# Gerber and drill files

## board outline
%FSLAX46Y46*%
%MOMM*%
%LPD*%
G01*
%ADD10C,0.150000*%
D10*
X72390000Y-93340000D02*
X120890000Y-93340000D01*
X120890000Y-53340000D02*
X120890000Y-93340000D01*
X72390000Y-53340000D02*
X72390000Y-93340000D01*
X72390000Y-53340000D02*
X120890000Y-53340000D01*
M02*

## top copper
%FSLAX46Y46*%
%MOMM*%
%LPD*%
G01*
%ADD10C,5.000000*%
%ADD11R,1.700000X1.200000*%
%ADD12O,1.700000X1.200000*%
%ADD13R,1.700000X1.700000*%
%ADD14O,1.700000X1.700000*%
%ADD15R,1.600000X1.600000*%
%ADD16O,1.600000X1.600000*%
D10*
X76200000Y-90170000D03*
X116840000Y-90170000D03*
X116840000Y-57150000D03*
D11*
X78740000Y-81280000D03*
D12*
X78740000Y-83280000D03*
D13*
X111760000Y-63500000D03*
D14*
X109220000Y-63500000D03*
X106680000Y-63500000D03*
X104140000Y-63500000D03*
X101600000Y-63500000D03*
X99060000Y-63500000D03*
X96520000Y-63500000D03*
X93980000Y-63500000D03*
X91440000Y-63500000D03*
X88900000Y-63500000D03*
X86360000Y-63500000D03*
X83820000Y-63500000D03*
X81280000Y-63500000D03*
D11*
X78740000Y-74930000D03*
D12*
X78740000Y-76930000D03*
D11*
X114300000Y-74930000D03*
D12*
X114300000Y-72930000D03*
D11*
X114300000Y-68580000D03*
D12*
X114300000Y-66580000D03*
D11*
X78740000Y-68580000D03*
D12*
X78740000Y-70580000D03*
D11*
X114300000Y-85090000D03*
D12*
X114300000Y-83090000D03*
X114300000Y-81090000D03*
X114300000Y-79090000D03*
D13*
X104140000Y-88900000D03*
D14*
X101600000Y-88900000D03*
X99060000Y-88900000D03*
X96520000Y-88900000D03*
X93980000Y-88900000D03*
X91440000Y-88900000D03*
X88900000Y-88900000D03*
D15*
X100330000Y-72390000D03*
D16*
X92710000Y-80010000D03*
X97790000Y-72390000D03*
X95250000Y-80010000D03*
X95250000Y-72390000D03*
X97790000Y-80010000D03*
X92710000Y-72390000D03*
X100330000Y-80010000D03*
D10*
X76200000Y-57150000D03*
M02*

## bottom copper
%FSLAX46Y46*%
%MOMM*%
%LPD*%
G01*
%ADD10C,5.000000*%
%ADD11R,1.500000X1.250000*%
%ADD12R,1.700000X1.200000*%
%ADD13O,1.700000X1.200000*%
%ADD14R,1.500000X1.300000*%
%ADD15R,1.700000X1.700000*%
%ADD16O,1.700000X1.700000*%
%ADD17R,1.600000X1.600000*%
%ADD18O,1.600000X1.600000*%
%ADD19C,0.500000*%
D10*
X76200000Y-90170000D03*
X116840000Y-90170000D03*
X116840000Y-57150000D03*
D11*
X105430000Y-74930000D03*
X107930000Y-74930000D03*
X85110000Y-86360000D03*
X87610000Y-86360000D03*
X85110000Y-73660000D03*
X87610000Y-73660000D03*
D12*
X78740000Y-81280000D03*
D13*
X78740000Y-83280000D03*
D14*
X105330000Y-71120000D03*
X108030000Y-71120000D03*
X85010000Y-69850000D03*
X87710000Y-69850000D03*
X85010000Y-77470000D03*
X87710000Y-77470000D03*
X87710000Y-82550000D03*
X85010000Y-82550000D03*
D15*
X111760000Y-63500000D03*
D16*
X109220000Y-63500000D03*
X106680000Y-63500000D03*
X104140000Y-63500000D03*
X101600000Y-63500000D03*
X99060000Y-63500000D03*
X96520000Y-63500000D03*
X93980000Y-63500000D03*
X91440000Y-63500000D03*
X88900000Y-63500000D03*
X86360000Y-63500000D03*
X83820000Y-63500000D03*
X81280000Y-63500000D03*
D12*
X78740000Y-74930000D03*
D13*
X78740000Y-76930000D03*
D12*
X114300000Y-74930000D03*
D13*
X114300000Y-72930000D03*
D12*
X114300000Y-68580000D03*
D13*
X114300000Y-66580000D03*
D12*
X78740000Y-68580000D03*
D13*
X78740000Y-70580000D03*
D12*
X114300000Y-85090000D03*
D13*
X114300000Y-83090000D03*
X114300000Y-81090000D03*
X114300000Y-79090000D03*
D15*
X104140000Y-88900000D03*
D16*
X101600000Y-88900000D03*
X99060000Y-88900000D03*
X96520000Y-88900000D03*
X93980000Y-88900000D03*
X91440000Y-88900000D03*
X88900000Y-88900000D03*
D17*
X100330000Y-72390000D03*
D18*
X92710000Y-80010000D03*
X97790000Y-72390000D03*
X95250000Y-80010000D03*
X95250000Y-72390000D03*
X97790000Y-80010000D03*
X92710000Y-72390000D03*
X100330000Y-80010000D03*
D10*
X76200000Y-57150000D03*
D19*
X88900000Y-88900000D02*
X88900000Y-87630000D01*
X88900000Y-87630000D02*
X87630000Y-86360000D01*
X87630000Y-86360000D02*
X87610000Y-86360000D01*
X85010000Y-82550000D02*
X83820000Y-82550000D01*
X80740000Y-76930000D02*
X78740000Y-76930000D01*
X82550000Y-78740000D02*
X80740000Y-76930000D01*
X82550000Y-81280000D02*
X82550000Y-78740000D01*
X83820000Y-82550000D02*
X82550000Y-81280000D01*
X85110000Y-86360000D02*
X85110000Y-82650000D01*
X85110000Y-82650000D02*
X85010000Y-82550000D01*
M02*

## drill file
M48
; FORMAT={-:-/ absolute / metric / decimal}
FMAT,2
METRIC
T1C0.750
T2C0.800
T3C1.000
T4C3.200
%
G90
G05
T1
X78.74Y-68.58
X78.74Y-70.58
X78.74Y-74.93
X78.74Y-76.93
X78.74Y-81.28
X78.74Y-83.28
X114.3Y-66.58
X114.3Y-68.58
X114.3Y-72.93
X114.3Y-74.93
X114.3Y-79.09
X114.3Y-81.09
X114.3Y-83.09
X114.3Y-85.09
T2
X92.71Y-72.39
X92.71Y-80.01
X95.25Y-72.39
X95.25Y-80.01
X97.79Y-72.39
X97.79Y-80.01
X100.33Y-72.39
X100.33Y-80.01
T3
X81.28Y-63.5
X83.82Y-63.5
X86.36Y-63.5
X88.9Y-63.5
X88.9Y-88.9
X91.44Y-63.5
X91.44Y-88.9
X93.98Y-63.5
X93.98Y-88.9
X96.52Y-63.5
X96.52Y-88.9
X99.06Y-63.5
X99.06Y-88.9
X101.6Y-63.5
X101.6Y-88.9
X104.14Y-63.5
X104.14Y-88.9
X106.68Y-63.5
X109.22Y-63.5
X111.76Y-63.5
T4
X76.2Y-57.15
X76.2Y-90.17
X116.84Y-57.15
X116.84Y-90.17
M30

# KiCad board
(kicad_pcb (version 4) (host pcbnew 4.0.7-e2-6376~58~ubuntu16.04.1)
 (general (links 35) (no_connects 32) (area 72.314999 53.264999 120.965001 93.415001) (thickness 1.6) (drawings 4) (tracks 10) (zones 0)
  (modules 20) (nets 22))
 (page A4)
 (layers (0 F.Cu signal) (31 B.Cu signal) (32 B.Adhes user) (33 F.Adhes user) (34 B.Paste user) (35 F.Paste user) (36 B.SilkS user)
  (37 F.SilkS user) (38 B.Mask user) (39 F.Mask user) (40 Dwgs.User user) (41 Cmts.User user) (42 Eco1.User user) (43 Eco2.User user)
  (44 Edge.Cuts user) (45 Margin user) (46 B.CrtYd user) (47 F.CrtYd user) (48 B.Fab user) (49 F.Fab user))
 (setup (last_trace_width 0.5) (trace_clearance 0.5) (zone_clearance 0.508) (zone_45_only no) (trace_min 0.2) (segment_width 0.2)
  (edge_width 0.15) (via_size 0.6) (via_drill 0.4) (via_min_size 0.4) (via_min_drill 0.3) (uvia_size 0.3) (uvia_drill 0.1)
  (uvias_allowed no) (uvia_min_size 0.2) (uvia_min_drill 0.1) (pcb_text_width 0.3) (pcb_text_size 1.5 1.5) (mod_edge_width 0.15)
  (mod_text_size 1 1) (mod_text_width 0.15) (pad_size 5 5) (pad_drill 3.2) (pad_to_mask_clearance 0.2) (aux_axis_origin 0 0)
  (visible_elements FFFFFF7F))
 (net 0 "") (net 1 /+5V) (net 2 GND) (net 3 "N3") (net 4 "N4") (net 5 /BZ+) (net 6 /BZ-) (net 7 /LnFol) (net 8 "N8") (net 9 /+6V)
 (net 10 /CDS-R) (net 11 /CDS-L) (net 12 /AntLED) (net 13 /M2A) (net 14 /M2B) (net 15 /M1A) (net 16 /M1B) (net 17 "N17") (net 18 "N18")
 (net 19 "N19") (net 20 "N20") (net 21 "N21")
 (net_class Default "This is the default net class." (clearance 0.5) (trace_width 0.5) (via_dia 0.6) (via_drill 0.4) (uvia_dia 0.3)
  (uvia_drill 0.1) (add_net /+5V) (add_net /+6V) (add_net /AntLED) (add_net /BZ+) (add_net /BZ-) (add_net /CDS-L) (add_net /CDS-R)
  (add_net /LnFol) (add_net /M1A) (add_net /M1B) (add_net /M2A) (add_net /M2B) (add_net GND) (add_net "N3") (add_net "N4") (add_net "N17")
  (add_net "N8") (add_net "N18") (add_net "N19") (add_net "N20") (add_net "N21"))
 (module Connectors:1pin (layer F.Cu) (at 76.2 90.17)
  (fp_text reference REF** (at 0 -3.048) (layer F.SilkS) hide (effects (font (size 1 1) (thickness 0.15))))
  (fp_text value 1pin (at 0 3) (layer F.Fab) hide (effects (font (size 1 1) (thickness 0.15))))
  (pad 1 thru_hole circle (at 0 0) (size 5 5) (drill 3.2) (layers *.Cu *.Mask)))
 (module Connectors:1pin (layer F.Cu) (at 116.84 90.17)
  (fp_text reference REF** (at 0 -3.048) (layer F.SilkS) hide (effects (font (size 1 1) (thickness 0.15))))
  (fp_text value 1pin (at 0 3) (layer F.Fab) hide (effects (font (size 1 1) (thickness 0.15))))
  (pad 1 thru_hole circle (at 0 0) (size 5 5) (drill 3.2) (layers *.Cu *.Mask)))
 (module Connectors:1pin (layer F.Cu) (at 116.84 57.15)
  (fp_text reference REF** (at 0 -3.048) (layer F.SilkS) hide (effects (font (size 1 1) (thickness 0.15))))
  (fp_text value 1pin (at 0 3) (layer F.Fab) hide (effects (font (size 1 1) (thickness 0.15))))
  (pad 1 thru_hole circle (at 0 0) (size 5 5) (drill 3.2) (layers *.Cu *.Mask)))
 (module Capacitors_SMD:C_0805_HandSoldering (layer B.Cu) (at 106.68 74.93)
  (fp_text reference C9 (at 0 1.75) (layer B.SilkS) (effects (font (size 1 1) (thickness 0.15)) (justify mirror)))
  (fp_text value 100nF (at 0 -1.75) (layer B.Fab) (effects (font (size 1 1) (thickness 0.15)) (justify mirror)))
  (pad 1 smd rect (at -1.25 0) (size 1.5 1.25) (layers B.Cu B.Paste B.Mask) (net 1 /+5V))
  (pad 2 smd rect (at 1.25 0) (size 1.5 1.25) (layers B.Cu B.Paste B.Mask) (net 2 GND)))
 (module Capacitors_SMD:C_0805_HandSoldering (layer B.Cu) (at 86.36 86.36)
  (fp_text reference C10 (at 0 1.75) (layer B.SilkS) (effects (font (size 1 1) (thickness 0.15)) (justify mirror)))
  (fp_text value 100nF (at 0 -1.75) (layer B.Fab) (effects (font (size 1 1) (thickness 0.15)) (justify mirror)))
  (pad 1 smd rect (at -1.25 0) (size 1.5 1.25) (layers B.Cu B.Paste B.Mask) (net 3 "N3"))
  (pad 2 smd rect (at 1.25 0) (size 1.5 1.25) (layers B.Cu B.Paste B.Mask) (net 2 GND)))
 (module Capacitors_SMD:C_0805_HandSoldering (layer B.Cu) (at 86.36 73.66)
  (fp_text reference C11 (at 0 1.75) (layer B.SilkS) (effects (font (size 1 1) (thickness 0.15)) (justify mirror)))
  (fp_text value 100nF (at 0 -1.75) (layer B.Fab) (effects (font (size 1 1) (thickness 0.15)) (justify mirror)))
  (pad 1 smd rect (at -1.25 0) (size 1.5 1.25) (layers B.Cu B.Paste B.Mask) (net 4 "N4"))
  (pad 2 smd rect (at 1.25 0) (size 1.5 1.25) (layers B.Cu B.Paste B.Mask) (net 2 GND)))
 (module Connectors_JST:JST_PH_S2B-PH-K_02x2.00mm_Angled (layer F.Cu) (at 78.74 81.28 270)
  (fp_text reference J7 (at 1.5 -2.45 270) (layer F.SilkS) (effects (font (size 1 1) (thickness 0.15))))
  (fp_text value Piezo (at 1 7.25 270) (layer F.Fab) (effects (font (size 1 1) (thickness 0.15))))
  (pad 1 thru_hole rect (at 0 0 270) (size 1.2 1.7) (drill 0.75) (layers *.Cu *.Mask) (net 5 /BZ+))
  (pad 2 thru_hole oval (at 2 0 270) (size 1.2 1.7) (drill 0.75) (layers *.Cu *.Mask) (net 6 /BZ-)))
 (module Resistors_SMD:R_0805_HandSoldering (layer B.Cu) (at 106.68 71.12)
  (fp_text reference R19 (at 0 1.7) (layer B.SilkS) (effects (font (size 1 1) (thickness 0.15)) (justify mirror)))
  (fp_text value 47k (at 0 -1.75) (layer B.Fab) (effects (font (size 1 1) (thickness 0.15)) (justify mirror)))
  (pad 1 smd rect (at -1.35 0) (size 1.5 1.3) (layers B.Cu B.Paste B.Mask) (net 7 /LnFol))
  (pad 2 smd rect (at 1.35 0) (size 1.5 1.3) (layers B.Cu B.Paste B.Mask) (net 1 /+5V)))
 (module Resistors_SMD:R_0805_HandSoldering (layer B.Cu) (at 86.36 69.85)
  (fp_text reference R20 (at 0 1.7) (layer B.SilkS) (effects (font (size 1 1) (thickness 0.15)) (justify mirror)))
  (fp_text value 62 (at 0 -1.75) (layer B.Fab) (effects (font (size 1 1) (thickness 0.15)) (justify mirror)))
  (pad 1 smd rect (at -1.35 0) (size 1.5 1.3) (layers B.Cu B.Paste B.Mask) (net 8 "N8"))
  (pad 2 smd rect (at 1.35 0) (size 1.5 1.3) (layers B.Cu B.Paste B.Mask) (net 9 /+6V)))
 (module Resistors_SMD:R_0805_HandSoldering (layer B.Cu) (at 86.36 77.47)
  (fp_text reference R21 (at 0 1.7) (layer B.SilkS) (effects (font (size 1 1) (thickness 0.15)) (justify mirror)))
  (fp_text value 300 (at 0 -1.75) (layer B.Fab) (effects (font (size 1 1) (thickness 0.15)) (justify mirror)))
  (pad 1 smd rect (at -1.35 0) (size 1.5 1.3) (layers B.Cu B.Paste B.Mask) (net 4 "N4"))
  (pad 2 smd rect (at 1.35 0) (size 1.5 1.3) (layers B.Cu B.Paste B.Mask) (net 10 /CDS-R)))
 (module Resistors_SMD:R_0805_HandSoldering (layer B.Cu) (at 86.36 82.55 180)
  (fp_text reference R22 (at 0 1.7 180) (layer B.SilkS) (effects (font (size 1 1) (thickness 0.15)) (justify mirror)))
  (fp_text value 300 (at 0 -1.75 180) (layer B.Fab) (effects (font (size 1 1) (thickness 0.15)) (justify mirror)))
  (pad 1 smd rect (at -1.35 0 180) (size 1.5 1.3) (layers B.Cu B.Paste B.Mask) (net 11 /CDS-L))
  (pad 2 smd rect (at 1.35 0 180) (size 1.5 1.3) (layers B.Cu B.Paste B.Mask) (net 3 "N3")))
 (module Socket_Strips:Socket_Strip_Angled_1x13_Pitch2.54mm (layer F.Cu) (at 111.76 63.5 270)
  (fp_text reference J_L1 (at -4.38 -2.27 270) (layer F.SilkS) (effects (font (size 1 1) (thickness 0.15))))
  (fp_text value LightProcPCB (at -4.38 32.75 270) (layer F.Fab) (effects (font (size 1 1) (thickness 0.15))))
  (pad 1 thru_hole rect (at 0 0 270) (size 1.7 1.7) (drill 1) (layers *.Cu *.Mask) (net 7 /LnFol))
  (pad 2 thru_hole oval (at 0 2.54 270) (size 1.7 1.7) (drill 1) (layers *.Cu *.Mask) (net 5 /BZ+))
  (pad 3 thru_hole oval (at 0 5.08 270) (size 1.7 1.7) (drill 1) (layers *.Cu *.Mask) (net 6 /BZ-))
  (pad 4 thru_hole oval (at 0 7.62 270) (size 1.7 1.7) (drill 1) (layers *.Cu *.Mask) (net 11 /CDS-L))
  (pad 5 thru_hole oval (at 0 10.16 270) (size 1.7 1.7) (drill 1) (layers *.Cu *.Mask) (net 10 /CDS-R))
  (pad 6 thru_hole oval (at 0 12.7 270) (size 1.7 1.7) (drill 1) (layers *.Cu *.Mask) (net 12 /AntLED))
  (pad 7 thru_hole oval (at 0 15.24 270) (size 1.7 1.7) (drill 1) (layers *.Cu *.Mask) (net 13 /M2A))
  (pad 8 thru_hole oval (at 0 17.78 270) (size 1.7 1.7) (drill 1) (layers *.Cu *.Mask) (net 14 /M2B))
  (pad 9 thru_hole oval (at 0 20.32 270) (size 1.7 1.7) (drill 1) (layers *.Cu *.Mask) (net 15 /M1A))
  (pad 10 thru_hole oval (at 0 22.86 270) (size 1.7 1.7) (drill 1) (layers *.Cu *.Mask) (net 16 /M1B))
  (pad 11 thru_hole oval (at 0 25.4 270) (size 1.7 1.7) (drill 1) (layers *.Cu *.Mask) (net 1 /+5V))
  (pad 12 thru_hole oval (at 0 27.94 270) (size 1.7 1.7) (drill 1) (layers *.Cu *.Mask) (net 9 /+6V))
  (pad 13 thru_hole oval (at 0 30.48 270) (size 1.7 1.7) (drill 1) (layers *.Cu *.Mask) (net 2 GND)))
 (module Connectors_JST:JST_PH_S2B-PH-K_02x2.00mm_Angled (layer F.Cu) (at 78.74 74.93 270)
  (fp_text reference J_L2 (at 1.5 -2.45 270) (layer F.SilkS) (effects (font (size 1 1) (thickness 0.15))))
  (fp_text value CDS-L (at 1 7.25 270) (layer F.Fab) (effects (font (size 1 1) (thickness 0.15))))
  (pad 1 thru_hole rect (at 0 0 270) (size 1.2 1.7) (drill 0.75) (layers *.Cu *.Mask) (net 1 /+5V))
  (pad 2 thru_hole oval (at 2 0 270) (size 1.2 1.7) (drill 0.75) (layers *.Cu *.Mask) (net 3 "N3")))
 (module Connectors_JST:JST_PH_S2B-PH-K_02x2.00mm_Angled (layer F.Cu) (at 114.3 74.93 90)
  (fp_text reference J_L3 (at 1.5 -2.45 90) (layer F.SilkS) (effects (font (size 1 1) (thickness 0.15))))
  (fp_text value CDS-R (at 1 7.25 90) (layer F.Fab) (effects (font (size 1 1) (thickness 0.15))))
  (pad 1 thru_hole rect (at 0 0 90) (size 1.2 1.7) (drill 0.75) (layers *.Cu *.Mask) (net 1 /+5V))
  (pad 2 thru_hole oval (at 2 0 90) (size 1.2 1.7) (drill 0.75) (layers *.Cu *.Mask) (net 4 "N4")))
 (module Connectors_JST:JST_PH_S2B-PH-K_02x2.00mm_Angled (layer F.Cu) (at 114.3 68.58 90)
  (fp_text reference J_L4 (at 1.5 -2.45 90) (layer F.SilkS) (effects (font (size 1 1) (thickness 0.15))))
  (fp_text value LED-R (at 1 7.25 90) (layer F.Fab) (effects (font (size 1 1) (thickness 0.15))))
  (pad 1 thru_hole rect (at 0 0 90) (size 1.2 1.7) (drill 0.75) (layers *.Cu *.Mask) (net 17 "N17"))
  (pad 2 thru_hole oval (at 2 0 90) (size 1.2 1.7) (drill 0.75) (layers *.Cu *.Mask) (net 12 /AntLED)))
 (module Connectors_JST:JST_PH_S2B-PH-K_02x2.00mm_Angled (layer F.Cu) (at 78.74 68.58 270)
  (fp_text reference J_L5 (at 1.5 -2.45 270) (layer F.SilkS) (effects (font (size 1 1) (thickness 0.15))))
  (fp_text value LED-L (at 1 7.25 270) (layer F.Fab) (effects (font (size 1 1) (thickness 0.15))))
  (pad 1 thru_hole rect (at 0 0 270) (size 1.2 1.7) (drill 0.75) (layers *.Cu *.Mask) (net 8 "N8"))
  (pad 2 thru_hole oval (at 2 0 270) (size 1.2 1.7) (drill 0.75) (layers *.Cu *.Mask) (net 17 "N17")))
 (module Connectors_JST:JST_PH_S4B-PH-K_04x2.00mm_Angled (layer F.Cu) (at 114.3 85.09 90)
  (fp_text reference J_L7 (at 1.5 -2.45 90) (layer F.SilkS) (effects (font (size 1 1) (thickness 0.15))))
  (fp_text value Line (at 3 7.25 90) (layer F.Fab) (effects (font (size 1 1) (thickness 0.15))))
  (pad 1 thru_hole rect (at 0 0 90) (size 1.2 1.7) (drill 0.75) (layers *.Cu *.Mask) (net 2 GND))
  (pad 2 thru_hole oval (at 2 0 90) (size 1.2 1.7) (drill 0.75) (layers *.Cu *.Mask) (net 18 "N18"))
  (pad 3 thru_hole oval (at 4 0 90) (size 1.2 1.7) (drill 0.75) (layers *.Cu *.Mask) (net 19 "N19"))
  (pad 4 thru_hole oval (at 6 0 90) (size 1.2 1.7) (drill 0.75) (layers *.Cu *.Mask) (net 1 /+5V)))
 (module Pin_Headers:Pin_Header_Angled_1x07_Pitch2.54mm (layer F.Cu) (at 104.14 88.9 270)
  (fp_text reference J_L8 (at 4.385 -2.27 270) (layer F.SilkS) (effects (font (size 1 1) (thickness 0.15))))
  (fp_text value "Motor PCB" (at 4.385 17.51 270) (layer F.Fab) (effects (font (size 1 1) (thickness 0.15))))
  (pad 1 thru_hole rect (at 0 0 270) (size 1.7 1.7) (drill 1) (layers *.Cu *.Mask) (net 13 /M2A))
  (pad 2 thru_hole oval (at 0 2.54 270) (size 1.7 1.7) (drill 1) (layers *.Cu *.Mask) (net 14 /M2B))
  (pad 3 thru_hole oval (at 0 5.08 270) (size 1.7 1.7) (drill 1) (layers *.Cu *.Mask) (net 15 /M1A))
  (pad 4 thru_hole oval (at 0 7.62 270) (size 1.7 1.7) (drill 1) (layers *.Cu *.Mask) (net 16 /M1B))
  (pad 5 thru_hole oval (at 0 10.16 270) (size 1.7 1.7) (drill 1) (layers *.Cu *.Mask) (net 1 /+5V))
  (pad 6 thru_hole oval (at 0 12.7 270) (size 1.7 1.7) (drill 1) (layers *.Cu *.Mask) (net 9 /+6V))
  (pad 7 thru_hole oval (at 0 15.24 270) (size 1.7 1.7) (drill 1) (layers *.Cu *.Mask) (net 2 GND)))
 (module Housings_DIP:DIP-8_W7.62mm (layer F.Cu) (at 100.33 72.39 270)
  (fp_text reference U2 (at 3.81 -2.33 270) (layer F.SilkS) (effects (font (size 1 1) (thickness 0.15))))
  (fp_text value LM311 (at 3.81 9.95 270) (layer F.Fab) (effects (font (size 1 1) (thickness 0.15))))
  (pad 1 thru_hole rect (at 0 0 270) (size 1.6 1.6) (drill 0.8) (layers *.Cu *.Mask) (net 2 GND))
  (pad 5 thru_hole oval (at 7.62 7.62 270) (size 1.6 1.6) (drill 0.8) (layers *.Cu *.Mask) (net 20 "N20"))
  (pad 2 thru_hole oval (at 0 2.54 270) (size 1.6 1.6) (drill 0.8) (layers *.Cu *.Mask) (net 19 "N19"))
  (pad 6 thru_hole oval (at 7.62 5.08 270) (size 1.6 1.6) (drill 0.8) (layers *.Cu *.Mask) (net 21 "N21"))
  (pad 3 thru_hole oval (at 0 5.08 270) (size 1.6 1.6) (drill 0.8) (layers *.Cu *.Mask) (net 18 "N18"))
  (pad 7 thru_hole oval (at 7.62 2.54 270) (size 1.6 1.6) (drill 0.8) (layers *.Cu *.Mask) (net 7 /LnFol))
  (pad 4 thru_hole oval (at 0 7.62 270) (size 1.6 1.6) (drill 0.8) (layers *.Cu *.Mask) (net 2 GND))
  (pad 8 thru_hole oval (at 7.62 0 270) (size 1.6 1.6) (drill 0.8) (layers *.Cu *.Mask) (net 1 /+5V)))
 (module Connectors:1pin (layer F.Cu) (at 76.2 57.15)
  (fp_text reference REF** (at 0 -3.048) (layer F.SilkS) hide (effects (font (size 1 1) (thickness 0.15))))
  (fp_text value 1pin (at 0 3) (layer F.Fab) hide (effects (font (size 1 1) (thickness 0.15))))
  (pad 1 thru_hole circle (at 0 0) (size 5 5) (drill 3.2) (layers *.Cu *.Mask)))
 (gr_line (start 72.39 93.34) (end 120.89 93.34) (angle 90) (layer Edge.Cuts) (width 0.15))
 (gr_line (start 120.89 53.34) (end 120.89 93.34) (angle 90) (layer Edge.Cuts) (width 0.15))
 (gr_line (start 72.39 53.34) (end 72.39 93.34) (angle 90) (layer Edge.Cuts) (width 0.15))
 (gr_line (start 72.39 53.34) (end 120.89 53.34) (angle 90) (layer Edge.Cuts) (width 0.15))
 (segment (start 88.9 88.9) (end 88.9 87.63) (width 0.5) (layer B.Cu) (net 2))
 (segment (start 88.9 87.63) (end 87.63 86.36) (width 0.5) (layer B.Cu) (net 2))
 (segment (start 87.63 86.36) (end 87.61 86.36) (width 0.5) (layer B.Cu) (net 2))
 (segment (start 85.01 82.55) (end 83.82 82.55) (width 0.5) (layer B.Cu) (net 3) (status 400000))
 (segment (start 80.74 76.93) (end 78.74 76.93) (width 0.5) (layer B.Cu) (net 3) (status 800000))
 (segment (start 82.55 78.74) (end 80.74 76.93) (width 0.5) (layer B.Cu) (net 3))
 (segment (start 82.55 81.28) (end 82.55 78.74) (width 0.5) (layer B.Cu) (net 3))
 (segment (start 83.82 82.55) (end 82.55 81.28) (width 0.5) (layer B.Cu) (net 3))
 (segment (start 85.11 86.36) (end 85.11 82.65) (width 0.5) (layer B.Cu) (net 3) (status C00000))
 (segment (start 85.11 82.65) (end 85.01 82.55) (width 0.5) (layer B.Cu) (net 3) (status C00000)))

